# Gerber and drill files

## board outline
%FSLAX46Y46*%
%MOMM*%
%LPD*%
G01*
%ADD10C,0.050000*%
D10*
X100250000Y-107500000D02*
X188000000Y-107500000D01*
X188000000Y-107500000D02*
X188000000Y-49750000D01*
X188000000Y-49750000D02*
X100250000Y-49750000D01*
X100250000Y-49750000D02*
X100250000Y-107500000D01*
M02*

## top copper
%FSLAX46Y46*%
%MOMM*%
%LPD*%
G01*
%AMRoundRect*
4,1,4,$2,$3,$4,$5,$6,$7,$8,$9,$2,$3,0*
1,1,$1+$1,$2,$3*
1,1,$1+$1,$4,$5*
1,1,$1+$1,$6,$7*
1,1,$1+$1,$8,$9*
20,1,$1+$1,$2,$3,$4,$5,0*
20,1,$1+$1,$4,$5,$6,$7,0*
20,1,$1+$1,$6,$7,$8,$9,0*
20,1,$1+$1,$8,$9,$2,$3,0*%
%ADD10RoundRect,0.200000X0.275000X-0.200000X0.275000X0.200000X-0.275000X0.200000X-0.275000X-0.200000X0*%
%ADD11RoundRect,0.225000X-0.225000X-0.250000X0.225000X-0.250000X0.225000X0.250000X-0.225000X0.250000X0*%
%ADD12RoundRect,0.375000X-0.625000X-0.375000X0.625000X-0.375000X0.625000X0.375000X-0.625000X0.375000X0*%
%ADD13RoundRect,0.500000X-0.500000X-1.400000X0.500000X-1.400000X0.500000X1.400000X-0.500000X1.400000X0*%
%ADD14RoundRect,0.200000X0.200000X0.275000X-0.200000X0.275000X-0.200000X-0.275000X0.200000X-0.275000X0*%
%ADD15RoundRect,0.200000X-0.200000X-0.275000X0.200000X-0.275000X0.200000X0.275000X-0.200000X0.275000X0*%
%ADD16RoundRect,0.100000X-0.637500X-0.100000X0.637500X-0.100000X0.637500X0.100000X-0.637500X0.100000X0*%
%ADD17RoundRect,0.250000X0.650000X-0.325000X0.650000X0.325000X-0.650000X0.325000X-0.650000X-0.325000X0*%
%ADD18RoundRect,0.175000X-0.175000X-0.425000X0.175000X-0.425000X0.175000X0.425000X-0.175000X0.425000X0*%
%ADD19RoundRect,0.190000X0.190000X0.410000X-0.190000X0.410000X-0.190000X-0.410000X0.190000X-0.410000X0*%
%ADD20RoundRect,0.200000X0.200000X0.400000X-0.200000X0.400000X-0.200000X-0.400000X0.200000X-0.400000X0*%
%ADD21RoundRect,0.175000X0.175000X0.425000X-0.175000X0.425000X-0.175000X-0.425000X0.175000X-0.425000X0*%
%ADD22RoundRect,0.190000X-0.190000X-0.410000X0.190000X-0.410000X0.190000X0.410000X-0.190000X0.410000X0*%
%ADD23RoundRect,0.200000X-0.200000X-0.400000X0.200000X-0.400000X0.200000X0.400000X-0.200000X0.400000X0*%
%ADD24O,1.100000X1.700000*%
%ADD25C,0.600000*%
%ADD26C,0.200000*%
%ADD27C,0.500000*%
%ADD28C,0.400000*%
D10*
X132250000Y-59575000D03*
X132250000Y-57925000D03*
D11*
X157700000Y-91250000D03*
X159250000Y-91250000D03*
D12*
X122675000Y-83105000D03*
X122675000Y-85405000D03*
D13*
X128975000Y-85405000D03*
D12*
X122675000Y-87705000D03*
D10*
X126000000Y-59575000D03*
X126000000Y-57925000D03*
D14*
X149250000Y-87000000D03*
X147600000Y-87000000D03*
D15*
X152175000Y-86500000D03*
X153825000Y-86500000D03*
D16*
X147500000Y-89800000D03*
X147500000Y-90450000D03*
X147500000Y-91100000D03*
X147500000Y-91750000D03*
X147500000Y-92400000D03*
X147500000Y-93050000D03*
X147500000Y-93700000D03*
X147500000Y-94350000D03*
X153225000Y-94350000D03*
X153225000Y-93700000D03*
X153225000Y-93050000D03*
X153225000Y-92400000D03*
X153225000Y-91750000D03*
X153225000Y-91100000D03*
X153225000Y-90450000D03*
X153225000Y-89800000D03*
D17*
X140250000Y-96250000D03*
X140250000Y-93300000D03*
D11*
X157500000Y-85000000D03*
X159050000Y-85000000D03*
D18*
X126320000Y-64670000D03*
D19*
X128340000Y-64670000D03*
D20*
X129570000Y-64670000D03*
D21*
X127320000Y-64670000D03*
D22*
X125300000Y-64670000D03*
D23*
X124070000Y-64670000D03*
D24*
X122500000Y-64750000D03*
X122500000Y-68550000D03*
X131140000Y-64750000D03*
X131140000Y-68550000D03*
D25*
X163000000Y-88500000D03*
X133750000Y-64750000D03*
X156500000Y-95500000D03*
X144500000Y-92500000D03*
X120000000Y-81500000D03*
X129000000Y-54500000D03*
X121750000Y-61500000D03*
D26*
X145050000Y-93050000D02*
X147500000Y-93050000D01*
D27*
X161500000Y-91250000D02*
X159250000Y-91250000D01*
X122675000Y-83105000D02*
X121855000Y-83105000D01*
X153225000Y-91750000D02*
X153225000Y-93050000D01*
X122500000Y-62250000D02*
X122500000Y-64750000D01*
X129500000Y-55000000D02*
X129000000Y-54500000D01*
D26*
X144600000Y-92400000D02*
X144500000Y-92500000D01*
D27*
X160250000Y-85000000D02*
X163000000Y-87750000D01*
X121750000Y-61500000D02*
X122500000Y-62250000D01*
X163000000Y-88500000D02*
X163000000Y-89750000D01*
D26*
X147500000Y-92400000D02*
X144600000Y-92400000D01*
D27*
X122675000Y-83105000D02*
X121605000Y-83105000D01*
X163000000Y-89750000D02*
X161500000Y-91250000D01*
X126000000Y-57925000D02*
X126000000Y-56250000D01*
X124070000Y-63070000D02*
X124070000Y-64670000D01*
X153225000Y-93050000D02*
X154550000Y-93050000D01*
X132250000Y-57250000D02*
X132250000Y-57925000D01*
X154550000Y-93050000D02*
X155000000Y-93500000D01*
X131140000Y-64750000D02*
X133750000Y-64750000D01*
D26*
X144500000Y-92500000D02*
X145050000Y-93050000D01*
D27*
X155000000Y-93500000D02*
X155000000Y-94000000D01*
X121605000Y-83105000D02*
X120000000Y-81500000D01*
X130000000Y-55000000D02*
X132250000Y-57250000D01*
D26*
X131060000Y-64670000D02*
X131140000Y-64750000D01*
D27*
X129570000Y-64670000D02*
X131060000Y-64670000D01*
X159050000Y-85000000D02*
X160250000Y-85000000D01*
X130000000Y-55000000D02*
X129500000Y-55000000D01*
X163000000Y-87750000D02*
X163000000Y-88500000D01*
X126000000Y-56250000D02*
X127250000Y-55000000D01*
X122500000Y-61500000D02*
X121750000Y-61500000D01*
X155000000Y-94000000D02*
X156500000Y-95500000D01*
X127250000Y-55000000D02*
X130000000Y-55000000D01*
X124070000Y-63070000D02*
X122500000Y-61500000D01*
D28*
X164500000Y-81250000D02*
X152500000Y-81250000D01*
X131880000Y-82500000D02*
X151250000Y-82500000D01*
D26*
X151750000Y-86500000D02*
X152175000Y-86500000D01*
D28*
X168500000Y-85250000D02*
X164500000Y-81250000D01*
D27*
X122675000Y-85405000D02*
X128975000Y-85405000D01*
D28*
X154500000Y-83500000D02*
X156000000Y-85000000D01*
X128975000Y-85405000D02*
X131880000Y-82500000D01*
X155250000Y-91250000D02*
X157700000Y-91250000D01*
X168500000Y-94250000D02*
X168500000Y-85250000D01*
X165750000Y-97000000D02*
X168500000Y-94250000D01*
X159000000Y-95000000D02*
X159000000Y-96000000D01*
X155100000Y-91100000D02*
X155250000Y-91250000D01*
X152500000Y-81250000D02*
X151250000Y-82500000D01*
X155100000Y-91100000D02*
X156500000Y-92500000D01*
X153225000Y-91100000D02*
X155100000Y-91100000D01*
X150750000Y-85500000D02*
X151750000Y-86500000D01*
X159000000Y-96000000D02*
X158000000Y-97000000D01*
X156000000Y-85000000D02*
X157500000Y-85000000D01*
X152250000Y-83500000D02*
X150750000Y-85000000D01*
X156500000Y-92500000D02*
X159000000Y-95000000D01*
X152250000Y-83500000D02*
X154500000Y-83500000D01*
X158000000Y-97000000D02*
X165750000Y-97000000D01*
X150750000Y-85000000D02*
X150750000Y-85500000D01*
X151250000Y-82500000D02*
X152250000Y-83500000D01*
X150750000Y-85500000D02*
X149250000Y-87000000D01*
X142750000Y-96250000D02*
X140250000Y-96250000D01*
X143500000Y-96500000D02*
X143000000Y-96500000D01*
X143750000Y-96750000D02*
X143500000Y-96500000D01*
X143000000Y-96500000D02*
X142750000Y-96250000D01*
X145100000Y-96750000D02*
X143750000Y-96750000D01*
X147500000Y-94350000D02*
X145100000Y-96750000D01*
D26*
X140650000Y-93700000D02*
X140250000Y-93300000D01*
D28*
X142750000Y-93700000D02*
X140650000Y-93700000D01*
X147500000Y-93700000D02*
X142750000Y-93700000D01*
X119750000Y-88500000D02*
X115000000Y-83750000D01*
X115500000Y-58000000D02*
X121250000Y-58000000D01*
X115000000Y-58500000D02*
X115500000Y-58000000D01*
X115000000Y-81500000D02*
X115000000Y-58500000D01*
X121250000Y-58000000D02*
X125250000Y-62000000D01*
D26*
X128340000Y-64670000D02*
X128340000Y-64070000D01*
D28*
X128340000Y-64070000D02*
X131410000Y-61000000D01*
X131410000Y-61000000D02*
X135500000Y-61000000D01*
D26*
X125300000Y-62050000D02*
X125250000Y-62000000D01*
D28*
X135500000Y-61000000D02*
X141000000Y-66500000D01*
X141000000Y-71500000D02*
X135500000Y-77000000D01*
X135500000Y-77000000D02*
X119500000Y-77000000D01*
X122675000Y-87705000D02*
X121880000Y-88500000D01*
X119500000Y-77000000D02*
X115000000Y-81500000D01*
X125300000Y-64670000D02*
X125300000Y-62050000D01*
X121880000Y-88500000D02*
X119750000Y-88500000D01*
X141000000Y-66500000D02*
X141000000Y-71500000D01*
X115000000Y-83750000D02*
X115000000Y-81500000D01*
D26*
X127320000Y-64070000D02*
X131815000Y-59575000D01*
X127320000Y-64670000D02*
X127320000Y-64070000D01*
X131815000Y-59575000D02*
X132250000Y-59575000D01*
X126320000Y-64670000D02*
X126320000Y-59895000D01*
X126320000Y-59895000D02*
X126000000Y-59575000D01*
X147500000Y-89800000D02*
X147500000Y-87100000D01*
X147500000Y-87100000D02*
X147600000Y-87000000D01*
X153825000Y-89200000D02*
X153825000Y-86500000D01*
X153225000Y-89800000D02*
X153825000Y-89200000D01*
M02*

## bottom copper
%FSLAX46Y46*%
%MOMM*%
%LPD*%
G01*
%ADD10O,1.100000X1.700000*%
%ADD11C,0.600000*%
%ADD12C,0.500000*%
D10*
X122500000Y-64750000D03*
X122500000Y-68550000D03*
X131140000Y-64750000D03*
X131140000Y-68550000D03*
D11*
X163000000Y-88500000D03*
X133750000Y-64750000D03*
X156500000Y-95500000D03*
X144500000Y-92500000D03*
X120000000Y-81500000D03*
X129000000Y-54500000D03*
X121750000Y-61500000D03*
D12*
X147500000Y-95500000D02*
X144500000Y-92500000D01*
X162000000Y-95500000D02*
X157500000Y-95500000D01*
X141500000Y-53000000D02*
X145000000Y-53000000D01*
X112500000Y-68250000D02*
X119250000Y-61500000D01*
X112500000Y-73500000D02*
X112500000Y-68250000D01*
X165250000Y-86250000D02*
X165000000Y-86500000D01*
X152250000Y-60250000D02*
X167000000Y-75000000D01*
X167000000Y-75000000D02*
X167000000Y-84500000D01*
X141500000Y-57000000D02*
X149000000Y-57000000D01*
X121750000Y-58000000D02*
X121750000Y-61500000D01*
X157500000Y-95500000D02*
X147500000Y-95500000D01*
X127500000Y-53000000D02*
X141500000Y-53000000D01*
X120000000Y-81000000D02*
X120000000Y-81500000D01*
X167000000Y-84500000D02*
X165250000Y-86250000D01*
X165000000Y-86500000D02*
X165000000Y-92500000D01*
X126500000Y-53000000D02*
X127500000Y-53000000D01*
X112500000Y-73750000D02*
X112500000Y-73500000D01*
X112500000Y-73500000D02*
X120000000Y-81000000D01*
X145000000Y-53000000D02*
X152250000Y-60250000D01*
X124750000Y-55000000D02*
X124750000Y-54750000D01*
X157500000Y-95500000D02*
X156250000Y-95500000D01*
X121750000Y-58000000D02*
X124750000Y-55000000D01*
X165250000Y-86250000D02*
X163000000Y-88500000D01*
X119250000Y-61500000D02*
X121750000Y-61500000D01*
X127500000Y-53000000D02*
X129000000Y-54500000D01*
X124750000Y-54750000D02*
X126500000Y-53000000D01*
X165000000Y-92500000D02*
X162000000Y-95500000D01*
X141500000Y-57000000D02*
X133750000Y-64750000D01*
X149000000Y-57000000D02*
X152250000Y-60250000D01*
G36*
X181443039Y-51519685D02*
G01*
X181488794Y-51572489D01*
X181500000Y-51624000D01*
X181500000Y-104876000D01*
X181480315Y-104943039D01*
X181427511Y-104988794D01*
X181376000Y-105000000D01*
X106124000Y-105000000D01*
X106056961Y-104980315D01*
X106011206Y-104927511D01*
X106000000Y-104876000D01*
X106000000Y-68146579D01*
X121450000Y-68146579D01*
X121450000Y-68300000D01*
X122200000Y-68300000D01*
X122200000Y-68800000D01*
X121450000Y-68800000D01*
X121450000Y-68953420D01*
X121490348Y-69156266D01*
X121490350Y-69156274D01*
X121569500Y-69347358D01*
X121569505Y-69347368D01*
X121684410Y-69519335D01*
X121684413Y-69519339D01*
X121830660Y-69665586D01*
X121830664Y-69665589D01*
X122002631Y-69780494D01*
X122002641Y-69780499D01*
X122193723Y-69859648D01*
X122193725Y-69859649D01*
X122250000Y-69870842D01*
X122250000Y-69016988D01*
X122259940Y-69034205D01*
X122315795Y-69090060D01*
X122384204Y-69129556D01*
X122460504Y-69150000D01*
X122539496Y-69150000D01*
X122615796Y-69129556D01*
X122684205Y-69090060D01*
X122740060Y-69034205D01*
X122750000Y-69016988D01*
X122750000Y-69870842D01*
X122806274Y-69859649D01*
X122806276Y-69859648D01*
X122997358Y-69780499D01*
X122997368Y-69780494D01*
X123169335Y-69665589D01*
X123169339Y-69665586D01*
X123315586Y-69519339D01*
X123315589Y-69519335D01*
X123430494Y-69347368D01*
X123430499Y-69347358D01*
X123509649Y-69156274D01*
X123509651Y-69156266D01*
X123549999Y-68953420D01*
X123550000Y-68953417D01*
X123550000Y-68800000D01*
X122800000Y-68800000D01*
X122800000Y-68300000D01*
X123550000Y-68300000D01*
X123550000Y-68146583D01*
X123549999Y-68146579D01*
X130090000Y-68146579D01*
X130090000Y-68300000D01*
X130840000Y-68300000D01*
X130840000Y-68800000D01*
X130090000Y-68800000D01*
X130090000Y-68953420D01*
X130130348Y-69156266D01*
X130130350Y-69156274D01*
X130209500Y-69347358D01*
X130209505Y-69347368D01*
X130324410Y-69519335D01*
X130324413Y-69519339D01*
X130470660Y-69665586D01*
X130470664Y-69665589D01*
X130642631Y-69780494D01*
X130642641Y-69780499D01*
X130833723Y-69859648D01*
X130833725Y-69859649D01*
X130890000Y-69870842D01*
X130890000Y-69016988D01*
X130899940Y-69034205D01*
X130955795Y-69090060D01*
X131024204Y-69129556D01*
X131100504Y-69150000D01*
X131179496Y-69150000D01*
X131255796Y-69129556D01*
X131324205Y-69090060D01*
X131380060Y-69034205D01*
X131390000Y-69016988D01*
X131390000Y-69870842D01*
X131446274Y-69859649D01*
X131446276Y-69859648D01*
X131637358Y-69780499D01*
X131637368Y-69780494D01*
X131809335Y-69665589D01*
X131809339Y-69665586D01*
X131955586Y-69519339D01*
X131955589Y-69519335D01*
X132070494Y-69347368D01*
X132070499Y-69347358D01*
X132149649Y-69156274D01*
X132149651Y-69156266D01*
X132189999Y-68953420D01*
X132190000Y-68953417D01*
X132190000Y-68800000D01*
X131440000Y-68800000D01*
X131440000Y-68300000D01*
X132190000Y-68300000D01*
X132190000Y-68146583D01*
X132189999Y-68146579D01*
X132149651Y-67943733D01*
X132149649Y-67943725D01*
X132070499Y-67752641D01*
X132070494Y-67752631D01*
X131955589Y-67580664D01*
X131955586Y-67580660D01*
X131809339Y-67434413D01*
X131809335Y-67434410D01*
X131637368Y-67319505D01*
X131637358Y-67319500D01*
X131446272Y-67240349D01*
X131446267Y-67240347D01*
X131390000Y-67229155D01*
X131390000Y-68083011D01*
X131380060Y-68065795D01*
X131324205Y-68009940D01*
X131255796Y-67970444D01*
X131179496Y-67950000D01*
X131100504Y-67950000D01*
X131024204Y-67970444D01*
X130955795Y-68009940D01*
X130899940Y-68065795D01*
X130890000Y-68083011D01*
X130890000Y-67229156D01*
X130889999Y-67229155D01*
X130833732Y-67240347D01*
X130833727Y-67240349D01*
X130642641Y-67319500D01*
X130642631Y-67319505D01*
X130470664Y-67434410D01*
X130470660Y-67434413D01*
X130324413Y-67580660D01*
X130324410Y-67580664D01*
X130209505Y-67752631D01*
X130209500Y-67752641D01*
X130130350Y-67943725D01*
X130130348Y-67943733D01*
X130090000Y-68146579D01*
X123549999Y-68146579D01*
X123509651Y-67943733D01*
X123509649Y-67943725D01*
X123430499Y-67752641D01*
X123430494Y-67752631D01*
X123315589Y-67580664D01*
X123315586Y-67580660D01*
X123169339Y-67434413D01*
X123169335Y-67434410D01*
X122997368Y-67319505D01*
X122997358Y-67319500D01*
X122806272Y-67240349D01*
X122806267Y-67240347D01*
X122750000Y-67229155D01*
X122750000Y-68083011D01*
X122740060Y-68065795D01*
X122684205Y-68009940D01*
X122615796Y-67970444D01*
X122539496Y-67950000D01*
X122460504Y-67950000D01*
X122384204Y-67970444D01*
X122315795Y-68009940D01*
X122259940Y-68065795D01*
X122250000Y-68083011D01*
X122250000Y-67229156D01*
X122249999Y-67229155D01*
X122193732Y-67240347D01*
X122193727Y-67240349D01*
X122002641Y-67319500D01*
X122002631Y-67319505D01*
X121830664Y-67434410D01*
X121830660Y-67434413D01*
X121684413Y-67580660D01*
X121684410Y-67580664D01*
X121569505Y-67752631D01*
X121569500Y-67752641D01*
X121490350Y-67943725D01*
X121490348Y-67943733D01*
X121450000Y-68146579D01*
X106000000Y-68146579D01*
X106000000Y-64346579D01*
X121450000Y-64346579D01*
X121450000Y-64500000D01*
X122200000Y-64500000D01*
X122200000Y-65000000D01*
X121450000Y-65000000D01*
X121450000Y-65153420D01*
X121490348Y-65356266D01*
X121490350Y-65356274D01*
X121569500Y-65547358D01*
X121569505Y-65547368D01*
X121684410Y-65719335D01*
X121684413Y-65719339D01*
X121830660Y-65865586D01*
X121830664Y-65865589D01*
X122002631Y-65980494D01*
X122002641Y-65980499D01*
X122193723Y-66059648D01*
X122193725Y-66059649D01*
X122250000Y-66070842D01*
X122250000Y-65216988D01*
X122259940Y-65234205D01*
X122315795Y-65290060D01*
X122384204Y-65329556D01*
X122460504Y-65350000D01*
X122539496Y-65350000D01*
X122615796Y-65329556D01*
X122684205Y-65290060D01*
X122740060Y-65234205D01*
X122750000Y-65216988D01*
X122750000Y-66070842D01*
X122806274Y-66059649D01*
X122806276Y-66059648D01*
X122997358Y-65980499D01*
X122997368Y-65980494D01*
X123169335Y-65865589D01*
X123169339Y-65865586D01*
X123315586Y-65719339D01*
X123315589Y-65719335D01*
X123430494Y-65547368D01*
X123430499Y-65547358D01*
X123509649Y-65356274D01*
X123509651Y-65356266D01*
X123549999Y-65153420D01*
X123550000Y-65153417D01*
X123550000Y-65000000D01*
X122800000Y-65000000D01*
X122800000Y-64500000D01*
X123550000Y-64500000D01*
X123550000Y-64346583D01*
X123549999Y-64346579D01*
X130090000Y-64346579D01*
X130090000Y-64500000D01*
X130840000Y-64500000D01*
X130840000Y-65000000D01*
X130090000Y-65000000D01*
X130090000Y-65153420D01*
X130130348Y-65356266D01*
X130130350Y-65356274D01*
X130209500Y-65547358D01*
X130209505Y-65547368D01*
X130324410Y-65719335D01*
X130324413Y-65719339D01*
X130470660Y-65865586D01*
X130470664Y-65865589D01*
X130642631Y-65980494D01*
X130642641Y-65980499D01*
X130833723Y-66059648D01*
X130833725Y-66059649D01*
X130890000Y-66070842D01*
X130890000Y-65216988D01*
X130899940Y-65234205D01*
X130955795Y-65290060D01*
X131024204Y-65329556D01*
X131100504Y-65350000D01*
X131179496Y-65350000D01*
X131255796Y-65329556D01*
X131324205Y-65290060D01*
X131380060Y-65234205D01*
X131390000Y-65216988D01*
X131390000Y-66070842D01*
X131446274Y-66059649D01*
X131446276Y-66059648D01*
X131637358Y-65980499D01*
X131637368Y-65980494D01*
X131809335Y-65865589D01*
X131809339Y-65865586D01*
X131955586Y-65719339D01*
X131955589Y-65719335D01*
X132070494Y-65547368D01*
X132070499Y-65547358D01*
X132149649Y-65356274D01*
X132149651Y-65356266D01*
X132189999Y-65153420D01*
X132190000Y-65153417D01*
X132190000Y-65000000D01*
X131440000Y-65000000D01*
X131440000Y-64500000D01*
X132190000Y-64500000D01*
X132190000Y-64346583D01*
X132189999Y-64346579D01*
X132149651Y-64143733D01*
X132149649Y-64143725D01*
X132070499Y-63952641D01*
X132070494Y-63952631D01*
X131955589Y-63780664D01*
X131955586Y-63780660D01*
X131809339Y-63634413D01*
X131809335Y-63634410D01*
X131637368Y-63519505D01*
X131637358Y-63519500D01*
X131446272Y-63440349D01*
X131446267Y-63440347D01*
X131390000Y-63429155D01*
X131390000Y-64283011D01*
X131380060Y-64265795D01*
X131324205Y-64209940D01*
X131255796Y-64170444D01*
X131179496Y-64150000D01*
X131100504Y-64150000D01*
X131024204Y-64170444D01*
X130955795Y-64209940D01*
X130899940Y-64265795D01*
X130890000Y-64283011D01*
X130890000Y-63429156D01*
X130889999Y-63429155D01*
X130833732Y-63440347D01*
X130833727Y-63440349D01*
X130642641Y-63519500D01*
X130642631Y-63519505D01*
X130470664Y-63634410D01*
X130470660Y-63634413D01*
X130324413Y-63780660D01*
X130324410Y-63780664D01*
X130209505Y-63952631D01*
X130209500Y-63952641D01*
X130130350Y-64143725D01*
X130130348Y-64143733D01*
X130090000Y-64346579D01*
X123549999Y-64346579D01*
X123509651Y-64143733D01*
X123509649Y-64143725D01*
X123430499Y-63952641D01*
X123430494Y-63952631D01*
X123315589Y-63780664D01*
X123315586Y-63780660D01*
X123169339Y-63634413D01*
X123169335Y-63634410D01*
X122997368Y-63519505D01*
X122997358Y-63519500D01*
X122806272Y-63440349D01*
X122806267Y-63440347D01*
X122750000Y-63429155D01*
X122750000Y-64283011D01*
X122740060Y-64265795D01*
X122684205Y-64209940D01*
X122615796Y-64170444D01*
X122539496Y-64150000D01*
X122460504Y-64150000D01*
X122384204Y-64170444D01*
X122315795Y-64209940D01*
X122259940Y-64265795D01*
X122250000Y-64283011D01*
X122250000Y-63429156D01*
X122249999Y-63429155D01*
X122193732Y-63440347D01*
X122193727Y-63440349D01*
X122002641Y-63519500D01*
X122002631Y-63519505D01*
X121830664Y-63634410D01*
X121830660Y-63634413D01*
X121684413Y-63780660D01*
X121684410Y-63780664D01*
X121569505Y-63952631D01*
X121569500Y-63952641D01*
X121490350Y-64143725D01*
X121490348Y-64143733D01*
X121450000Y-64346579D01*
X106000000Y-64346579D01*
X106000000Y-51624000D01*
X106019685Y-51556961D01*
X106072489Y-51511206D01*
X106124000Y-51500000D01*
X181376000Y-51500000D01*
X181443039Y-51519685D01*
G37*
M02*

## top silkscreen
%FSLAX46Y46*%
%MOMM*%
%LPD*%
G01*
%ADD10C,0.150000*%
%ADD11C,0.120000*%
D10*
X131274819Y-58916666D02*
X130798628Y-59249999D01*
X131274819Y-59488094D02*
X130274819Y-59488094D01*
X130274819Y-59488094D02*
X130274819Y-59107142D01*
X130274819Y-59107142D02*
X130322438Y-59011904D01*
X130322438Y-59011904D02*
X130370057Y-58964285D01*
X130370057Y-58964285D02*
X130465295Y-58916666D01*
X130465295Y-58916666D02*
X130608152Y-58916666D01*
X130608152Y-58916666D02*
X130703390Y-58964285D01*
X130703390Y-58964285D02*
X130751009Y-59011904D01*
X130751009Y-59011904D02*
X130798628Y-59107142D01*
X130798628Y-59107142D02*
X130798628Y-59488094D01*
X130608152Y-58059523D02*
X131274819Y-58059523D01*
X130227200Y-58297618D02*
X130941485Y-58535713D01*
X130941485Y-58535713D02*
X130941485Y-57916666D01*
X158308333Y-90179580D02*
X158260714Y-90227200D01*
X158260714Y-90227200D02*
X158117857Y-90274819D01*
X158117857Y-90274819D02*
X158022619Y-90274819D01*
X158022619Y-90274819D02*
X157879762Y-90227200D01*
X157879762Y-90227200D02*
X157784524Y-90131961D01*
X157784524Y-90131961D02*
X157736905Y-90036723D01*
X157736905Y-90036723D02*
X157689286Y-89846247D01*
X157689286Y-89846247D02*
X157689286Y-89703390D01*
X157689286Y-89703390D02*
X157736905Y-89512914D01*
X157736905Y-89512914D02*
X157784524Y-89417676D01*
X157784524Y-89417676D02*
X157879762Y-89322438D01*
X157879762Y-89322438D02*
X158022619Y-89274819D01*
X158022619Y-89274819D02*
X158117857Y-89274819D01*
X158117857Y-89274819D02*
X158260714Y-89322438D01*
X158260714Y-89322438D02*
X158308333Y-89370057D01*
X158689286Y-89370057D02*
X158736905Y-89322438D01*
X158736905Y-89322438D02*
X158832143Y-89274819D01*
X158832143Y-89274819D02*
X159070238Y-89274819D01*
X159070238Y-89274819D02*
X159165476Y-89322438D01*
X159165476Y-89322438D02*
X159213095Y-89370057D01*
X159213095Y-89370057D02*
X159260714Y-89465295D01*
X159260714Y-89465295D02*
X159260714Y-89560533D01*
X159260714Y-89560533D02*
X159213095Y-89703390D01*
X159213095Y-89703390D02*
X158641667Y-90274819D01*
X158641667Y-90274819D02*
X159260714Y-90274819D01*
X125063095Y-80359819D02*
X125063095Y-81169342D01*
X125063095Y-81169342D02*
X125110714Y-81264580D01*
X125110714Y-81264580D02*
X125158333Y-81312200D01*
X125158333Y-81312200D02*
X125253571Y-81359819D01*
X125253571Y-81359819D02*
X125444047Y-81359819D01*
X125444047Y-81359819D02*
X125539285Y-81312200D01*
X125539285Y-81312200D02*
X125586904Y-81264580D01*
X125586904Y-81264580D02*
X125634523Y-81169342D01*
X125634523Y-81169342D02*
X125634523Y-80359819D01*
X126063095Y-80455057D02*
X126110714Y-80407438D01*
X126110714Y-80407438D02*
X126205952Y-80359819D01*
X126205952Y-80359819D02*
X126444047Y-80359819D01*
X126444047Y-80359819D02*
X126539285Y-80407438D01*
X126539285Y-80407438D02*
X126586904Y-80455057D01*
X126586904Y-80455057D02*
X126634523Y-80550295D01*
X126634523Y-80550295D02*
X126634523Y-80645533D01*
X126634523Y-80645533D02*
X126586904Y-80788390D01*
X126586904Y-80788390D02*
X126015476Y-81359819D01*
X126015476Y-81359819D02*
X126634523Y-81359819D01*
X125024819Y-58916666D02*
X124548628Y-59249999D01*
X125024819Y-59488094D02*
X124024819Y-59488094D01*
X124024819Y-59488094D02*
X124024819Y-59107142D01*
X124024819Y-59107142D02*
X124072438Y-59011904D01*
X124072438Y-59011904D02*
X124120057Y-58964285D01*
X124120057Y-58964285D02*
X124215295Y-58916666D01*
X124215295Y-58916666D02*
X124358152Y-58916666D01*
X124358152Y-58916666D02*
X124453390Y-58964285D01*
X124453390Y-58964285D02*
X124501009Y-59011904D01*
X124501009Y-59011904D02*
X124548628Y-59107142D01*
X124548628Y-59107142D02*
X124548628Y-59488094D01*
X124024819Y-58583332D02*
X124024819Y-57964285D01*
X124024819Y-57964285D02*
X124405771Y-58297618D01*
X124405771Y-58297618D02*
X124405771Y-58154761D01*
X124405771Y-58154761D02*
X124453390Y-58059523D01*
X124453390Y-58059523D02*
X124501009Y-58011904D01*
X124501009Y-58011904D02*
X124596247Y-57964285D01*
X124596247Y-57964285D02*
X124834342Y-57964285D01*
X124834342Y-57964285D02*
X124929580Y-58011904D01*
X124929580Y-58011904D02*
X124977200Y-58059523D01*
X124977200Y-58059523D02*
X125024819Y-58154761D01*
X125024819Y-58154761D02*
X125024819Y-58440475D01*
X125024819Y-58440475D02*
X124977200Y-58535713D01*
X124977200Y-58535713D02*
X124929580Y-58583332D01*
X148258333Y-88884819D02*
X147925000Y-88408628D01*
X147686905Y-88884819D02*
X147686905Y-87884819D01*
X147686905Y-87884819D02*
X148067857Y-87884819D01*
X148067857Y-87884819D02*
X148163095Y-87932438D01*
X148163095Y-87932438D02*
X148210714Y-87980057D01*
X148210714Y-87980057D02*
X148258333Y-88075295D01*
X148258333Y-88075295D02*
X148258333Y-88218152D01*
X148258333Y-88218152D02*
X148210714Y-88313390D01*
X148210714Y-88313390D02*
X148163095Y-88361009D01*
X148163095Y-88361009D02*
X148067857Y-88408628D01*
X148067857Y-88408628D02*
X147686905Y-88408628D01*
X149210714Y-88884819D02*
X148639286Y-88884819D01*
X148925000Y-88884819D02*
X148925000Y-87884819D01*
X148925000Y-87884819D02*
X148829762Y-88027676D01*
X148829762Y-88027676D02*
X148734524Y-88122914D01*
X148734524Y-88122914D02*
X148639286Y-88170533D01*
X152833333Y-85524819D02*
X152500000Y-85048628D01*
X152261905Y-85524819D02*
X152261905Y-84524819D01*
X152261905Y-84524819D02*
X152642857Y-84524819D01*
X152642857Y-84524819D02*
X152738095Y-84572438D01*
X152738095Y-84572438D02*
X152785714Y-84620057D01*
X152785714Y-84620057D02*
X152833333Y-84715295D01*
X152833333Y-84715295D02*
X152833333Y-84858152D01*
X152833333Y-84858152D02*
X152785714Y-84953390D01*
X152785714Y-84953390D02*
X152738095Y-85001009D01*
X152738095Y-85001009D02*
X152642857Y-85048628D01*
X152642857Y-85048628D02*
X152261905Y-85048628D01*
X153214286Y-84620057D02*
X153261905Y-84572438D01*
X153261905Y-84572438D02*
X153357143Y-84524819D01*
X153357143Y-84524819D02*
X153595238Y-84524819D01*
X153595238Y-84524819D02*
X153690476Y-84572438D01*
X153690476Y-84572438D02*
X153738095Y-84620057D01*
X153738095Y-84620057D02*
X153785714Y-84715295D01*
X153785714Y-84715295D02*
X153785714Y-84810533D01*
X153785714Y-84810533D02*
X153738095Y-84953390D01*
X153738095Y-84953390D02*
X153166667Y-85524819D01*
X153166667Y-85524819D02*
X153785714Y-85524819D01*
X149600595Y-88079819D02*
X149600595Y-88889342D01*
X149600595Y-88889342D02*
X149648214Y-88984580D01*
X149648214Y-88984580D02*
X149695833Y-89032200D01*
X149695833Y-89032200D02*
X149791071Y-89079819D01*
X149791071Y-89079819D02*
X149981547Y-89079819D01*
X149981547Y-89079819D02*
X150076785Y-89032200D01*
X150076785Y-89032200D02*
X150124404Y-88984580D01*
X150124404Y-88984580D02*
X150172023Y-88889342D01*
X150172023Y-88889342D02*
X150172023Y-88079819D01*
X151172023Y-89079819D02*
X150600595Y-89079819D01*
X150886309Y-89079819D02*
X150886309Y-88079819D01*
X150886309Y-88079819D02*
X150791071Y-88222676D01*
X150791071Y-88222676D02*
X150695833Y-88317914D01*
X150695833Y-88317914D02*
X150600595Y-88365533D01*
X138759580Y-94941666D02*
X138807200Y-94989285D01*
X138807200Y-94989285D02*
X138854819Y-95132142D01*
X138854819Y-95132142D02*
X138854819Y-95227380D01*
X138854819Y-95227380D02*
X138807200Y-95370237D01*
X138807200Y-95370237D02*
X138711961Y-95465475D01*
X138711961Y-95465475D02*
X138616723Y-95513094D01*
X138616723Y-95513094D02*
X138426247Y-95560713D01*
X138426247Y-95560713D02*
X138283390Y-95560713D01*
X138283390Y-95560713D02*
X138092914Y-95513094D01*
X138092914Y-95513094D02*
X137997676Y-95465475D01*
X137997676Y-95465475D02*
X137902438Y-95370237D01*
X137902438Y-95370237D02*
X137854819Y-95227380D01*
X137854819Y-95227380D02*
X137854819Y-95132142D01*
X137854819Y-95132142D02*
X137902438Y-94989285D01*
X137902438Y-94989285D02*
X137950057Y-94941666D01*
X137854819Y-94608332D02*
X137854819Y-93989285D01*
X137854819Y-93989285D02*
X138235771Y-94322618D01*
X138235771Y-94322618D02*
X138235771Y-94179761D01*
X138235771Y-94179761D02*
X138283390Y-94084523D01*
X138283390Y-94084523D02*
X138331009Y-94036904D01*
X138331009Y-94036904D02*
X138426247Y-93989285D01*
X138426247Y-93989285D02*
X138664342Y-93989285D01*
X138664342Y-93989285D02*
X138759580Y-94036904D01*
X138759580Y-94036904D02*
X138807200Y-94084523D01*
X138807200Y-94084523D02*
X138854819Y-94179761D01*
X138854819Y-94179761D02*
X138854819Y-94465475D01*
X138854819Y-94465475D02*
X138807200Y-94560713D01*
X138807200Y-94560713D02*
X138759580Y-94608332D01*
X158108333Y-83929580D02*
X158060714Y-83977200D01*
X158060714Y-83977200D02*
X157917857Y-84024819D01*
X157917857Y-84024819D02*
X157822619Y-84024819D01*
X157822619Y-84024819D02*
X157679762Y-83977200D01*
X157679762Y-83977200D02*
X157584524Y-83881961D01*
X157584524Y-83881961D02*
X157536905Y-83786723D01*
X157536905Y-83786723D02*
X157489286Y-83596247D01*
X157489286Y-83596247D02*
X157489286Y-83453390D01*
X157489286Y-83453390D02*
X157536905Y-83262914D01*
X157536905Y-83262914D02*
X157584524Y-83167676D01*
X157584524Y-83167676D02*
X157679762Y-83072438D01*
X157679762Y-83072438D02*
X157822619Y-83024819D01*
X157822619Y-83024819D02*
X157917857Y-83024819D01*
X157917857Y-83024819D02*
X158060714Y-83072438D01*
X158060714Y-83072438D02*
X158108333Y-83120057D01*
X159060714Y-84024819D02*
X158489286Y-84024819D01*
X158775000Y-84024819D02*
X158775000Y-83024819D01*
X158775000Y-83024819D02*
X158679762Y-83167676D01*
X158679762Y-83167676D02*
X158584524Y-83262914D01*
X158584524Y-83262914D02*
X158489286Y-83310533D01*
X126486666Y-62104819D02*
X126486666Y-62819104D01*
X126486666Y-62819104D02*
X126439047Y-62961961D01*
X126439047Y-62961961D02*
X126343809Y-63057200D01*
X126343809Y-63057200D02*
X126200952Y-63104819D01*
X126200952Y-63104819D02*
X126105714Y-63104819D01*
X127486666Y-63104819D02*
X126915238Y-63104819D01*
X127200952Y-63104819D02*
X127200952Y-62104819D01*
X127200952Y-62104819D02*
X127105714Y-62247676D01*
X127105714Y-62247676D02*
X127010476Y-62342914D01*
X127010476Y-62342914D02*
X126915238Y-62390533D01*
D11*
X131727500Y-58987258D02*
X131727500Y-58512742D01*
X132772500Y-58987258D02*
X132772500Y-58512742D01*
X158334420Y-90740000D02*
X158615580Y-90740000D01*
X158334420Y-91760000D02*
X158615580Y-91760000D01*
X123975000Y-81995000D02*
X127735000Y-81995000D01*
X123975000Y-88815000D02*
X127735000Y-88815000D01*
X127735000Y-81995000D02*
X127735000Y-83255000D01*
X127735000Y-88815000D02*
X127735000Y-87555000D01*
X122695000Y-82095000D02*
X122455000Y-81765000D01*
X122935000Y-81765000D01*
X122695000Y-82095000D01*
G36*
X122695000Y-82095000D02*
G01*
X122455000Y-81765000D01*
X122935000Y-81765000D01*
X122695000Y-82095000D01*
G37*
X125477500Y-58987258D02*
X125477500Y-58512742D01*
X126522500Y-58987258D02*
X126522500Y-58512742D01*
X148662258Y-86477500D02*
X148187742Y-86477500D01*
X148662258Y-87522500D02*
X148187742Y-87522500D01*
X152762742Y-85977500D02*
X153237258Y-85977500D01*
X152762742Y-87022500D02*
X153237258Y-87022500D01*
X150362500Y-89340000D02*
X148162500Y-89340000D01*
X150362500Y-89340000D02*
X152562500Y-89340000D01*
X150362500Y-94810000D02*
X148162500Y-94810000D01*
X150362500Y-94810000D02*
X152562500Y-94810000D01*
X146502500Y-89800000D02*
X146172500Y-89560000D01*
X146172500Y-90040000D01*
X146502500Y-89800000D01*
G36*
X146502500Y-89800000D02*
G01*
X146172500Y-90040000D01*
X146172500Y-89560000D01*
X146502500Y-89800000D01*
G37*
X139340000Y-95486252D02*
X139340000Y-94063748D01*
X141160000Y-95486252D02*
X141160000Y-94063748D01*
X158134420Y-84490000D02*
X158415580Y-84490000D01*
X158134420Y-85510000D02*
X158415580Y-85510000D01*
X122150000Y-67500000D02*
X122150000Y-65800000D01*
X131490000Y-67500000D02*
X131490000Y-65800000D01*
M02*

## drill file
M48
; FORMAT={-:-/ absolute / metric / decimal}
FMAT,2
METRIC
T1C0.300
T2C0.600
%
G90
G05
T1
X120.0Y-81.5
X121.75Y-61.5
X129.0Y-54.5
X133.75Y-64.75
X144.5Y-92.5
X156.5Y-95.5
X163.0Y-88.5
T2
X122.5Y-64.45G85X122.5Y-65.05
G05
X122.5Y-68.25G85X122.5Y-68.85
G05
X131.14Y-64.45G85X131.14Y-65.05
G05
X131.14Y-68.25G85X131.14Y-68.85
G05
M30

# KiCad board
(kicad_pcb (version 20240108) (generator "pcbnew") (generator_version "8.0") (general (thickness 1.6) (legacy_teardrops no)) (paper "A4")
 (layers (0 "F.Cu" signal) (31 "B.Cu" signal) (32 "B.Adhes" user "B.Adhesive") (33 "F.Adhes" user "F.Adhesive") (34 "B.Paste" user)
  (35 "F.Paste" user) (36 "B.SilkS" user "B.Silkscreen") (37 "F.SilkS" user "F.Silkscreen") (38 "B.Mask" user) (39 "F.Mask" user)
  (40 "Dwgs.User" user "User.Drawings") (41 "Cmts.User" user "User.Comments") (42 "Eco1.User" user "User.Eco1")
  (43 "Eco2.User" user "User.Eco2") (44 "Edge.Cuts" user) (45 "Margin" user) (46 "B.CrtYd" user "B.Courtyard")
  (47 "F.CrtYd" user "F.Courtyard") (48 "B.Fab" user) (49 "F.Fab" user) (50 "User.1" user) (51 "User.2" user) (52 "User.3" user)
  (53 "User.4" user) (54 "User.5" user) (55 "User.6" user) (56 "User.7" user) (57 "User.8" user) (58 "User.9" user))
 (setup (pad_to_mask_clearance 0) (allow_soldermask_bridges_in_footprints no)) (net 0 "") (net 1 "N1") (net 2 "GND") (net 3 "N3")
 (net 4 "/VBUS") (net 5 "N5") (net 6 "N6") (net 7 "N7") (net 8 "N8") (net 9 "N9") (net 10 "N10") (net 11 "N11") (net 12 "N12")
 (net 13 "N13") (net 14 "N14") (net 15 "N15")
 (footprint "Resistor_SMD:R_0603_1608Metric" (layer "F.Cu") (at 132.25 58.75 90)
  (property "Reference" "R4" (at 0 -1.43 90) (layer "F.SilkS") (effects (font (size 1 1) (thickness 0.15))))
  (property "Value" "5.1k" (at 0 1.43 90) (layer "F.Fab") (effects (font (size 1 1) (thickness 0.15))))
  (fp_line (start -0.237258 -0.5225) (end 0.237258 -0.5225) (stroke (width 0.12) (type solid)) (layer "F.SilkS"))
  (fp_line (start -0.237258 0.5225) (end 0.237258 0.5225) (stroke (width 0.12) (type solid)) (layer "F.SilkS"))
  (pad "1" smd roundrect (at -0.825 0 90) (size 0.8 0.95) (layers "F.Cu" "F.Paste" "F.Mask") (roundrect_rratio 0.25) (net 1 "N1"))
  (pad "2" smd roundrect (at 0.825 0 90) (size 0.8 0.95) (layers "F.Cu" "F.Paste" "F.Mask") (roundrect_rratio 0.25) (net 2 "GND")))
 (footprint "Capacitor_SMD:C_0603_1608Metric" (layer "F.Cu") (at 158.475 91.25)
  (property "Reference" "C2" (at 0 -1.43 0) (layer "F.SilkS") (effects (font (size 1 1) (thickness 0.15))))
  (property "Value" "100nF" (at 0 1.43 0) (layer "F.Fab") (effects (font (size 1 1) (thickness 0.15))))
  (fp_line (start -0.14058 -0.51) (end 0.14058 -0.51) (stroke (width 0.12) (type solid)) (layer "F.SilkS"))
  (fp_line (start -0.14058 0.51) (end 0.14058 0.51) (stroke (width 0.12) (type solid)) (layer "F.SilkS"))
  (pad "1" smd roundrect (at -0.775 0) (size 0.9 0.95) (layers "F.Cu" "F.Paste" "F.Mask") (roundrect_rratio 0.25) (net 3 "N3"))
  (pad "2" smd roundrect (at 0.775 0) (size 0.9 0.95) (layers "F.Cu" "F.Paste" "F.Mask") (roundrect_rratio 0.25) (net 2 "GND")))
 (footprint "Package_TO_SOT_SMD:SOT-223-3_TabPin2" (layer "F.Cu") (at 125.825 85.405)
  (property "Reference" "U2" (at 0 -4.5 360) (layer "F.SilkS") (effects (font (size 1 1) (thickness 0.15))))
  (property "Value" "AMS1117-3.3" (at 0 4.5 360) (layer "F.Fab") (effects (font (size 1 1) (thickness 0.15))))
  (fp_line (start -1.85 -3.41) (end 1.91 -3.41) (stroke (width 0.12) (type solid)) (layer "F.SilkS"))
  (fp_line (start -1.85 3.41) (end 1.91 3.41) (stroke (width 0.12) (type solid)) (layer "F.SilkS"))
  (fp_line (start 1.91 -3.41) (end 1.91 -2.15) (stroke (width 0.12) (type solid)) (layer "F.SilkS"))
  (fp_line (start 1.91 3.41) (end 1.91 2.15) (stroke (width 0.12) (type solid)) (layer "F.SilkS"))
  (fp_poly
   (pts (xy -3.13 -3.31) (xy -3.37 -3.64) (xy -2.89 -3.64) (xy -3.13 -3.31)) (stroke (width 0.12) (type solid)) (fill solid)
   (layer "F.SilkS"))
  (pad "1" smd roundrect (at -3.15 -2.3) (size 2 1.5) (layers "F.Cu" "F.Paste" "F.Mask") (roundrect_rratio 0.25) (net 2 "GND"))
  (pad "2" smd roundrect (at -3.15 0) (size 2 1.5) (layers "F.Cu" "F.Paste" "F.Mask") (roundrect_rratio 0.25) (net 3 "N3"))
  (pad "2" smd roundrect (at 3.15 0) (size 2 3.8) (layers "F.Cu" "F.Paste" "F.Mask") (roundrect_rratio 0.25) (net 3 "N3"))
  (pad "3" smd roundrect (at -3.15 2.3) (size 2 1.5) (layers "F.Cu" "F.Paste" "F.Mask") (roundrect_rratio 0.25) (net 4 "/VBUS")))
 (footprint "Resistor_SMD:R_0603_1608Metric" (layer "F.Cu") (at 126 58.75 90)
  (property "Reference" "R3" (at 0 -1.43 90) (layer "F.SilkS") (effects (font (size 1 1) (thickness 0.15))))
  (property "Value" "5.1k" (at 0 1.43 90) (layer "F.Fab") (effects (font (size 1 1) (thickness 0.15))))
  (fp_line (start -0.237258 -0.5225) (end 0.237258 -0.5225) (stroke (width 0.12) (type solid)) (layer "F.SilkS"))
  (fp_line (start -0.237258 0.5225) (end 0.237258 0.5225) (stroke (width 0.12) (type solid)) (layer "F.SilkS"))
  (pad "1" smd roundrect (at -0.825 0 90) (size 0.8 0.95) (layers "F.Cu" "F.Paste" "F.Mask") (roundrect_rratio 0.25) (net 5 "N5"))
  (pad "2" smd roundrect (at 0.825 0 90) (size 0.8 0.95) (layers "F.Cu" "F.Paste" "F.Mask") (roundrect_rratio 0.25) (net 2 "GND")))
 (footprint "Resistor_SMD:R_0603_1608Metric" (layer "F.Cu") (at 148.425 87 180)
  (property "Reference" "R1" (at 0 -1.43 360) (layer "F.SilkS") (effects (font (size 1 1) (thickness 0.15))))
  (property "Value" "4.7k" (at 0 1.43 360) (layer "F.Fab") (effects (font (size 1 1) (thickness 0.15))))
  (fp_line (start -0.237258 0.5225) (end 0.237258 0.5225) (stroke (width 0.12) (type solid)) (layer "F.SilkS"))
  (fp_line (start -0.237258 -0.5225) (end 0.237258 -0.5225) (stroke (width 0.12) (type solid)) (layer "F.SilkS"))
  (pad "1" smd roundrect (at -0.825 0 180) (size 0.8 0.95) (layers "F.Cu" "F.Paste" "F.Mask") (roundrect_rratio 0.25) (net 3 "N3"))
  (pad "2" smd roundrect (at 0.825 0 180) (size 0.8 0.95) (layers "F.Cu" "F.Paste" "F.Mask") (roundrect_rratio 0.25) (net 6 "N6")))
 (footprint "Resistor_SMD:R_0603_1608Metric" (layer "F.Cu") (at 153 86.5)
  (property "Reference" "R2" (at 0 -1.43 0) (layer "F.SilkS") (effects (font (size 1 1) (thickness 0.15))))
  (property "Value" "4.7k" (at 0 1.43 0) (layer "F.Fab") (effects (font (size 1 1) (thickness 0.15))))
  (fp_line (start -0.237258 -0.5225) (end 0.237258 -0.5225) (stroke (width 0.12) (type solid)) (layer "F.SilkS"))
  (fp_line (start -0.237258 0.5225) (end 0.237258 0.5225) (stroke (width 0.12) (type solid)) (layer "F.SilkS"))
  (pad "1" smd roundrect (at -0.825 0) (size 0.8 0.95) (layers "F.Cu" "F.Paste" "F.Mask") (roundrect_rratio 0.25) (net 3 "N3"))
  (pad "2" smd roundrect (at 0.825 0) (size 0.8 0.95) (layers "F.Cu" "F.Paste" "F.Mask") (roundrect_rratio 0.25) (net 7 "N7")))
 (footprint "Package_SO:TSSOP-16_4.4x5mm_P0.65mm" (layer "F.Cu") (at 150.3625 92.075)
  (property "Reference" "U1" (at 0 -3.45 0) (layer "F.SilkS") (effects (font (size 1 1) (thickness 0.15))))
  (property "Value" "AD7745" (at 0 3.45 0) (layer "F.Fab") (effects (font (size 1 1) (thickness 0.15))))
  (fp_line (start 0 -2.735) (end -2.2 -2.735) (stroke (width 0.12) (type solid)) (layer "F.SilkS"))
  (fp_line (start 0 -2.735) (end 2.2 -2.735) (stroke (width 0.12) (type solid)) (layer "F.SilkS"))
  (fp_line (start 0 2.735) (end -2.2 2.735) (stroke (width 0.12) (type solid)) (layer "F.SilkS"))
  (fp_line (start 0 2.735) (end 2.2 2.735) (stroke (width 0.12) (type solid)) (layer "F.SilkS"))
  (fp_poly
   (pts (xy -3.86 -2.275) (xy -4.19 -2.515) (xy -4.19 -2.035) (xy -3.86 -2.275)) (stroke (width 0.12) (type solid)) (fill solid)
   (layer "F.SilkS"))
  (pad "1" smd roundrect (at -2.8625 -2.275) (size 1.475 0.4) (layers "F.Cu" "F.Paste" "F.Mask") (roundrect_rratio 0.25) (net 6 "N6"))
  (pad "2" smd roundrect (at -2.8625 -1.625) (size 1.475 0.4) (layers "F.Cu" "F.Paste" "F.Mask") (roundrect_rratio 0.25) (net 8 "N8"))
  (pad "3" smd roundrect (at -2.8625 -0.975) (size 1.475 0.4) (layers "F.Cu" "F.Paste" "F.Mask") (roundrect_rratio 0.25) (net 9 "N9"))
  (pad "4" smd roundrect (at -2.8625 -0.325) (size 1.475 0.4) (layers "F.Cu" "F.Paste" "F.Mask") (roundrect_rratio 0.25) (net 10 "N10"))
  (pad "5" smd roundrect (at -2.8625 0.325) (size 1.475 0.4) (layers "F.Cu" "F.Paste" "F.Mask") (roundrect_rratio 0.25) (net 2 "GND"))
  (pad "6" smd roundrect (at -2.8625 0.975) (size 1.475 0.4) (layers "F.Cu" "F.Paste" "F.Mask") (roundrect_rratio 0.25) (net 2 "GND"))
  (pad "7" smd roundrect (at -2.8625 1.625) (size 1.475 0.4) (layers "F.Cu" "F.Paste" "F.Mask") (roundrect_rratio 0.25) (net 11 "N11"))
  (pad "8" smd roundrect (at -2.8625 2.275) (size 1.475 0.4) (layers "F.Cu" "F.Paste" "F.Mask") (roundrect_rratio 0.25) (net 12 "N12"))
  (pad "9" smd roundrect (at 2.8625 2.275) (size 1.475 0.4) (layers "F.Cu" "F.Paste" "F.Mask") (roundrect_rratio 0.25) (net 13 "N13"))
  (pad "10" smd roundrect (at 2.8625 1.625) (size 1.475 0.4) (layers "F.Cu" "F.Paste" "F.Mask") (roundrect_rratio 0.25) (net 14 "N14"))
  (pad "11" smd roundrect (at 2.8625 0.975) (size 1.475 0.4) (layers "F.Cu" "F.Paste" "F.Mask") (roundrect_rratio 0.25) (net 2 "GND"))
  (pad "12" smd roundrect (at 2.8625 0.325) (size 1.475 0.4) (layers "F.Cu" "F.Paste" "F.Mask") (roundrect_rratio 0.25) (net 2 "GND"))
  (pad "13" smd roundrect (at 2.8625 -0.325) (size 1.475 0.4) (layers "F.Cu" "F.Paste" "F.Mask") (roundrect_rratio 0.25) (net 2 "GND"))
  (pad "14" smd roundrect (at 2.8625 -0.975) (size 1.475 0.4) (layers "F.Cu" "F.Paste" "F.Mask") (roundrect_rratio 0.25) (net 3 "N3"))
  (pad "15" smd roundrect (at 2.8625 -1.625) (size 1.475 0.4) (layers "F.Cu" "F.Paste" "F.Mask") (roundrect_rratio 0.25) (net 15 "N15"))
  (pad "16" smd roundrect (at 2.8625 -2.275) (size 1.475 0.4) (layers "F.Cu" "F.Paste" "F.Mask") (roundrect_rratio 0.25) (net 7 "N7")))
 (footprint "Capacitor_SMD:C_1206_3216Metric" (layer "F.Cu") (at 140.25 94.775 90)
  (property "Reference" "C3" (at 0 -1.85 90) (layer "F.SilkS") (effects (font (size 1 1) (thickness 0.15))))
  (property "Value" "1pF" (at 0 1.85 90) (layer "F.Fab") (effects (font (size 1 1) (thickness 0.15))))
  (fp_line (start -0.711252 -0.91) (end 0.711252 -0.91) (stroke (width 0.12) (type solid)) (layer "F.SilkS"))
  (fp_line (start -0.711252 0.91) (end 0.711252 0.91) (stroke (width 0.12) (type solid)) (layer "F.SilkS"))
  (pad "1" smd roundrect (at -1.475 0 90) (size 1.15 1.8) (layers "F.Cu" "F.Paste" "F.Mask") (roundrect_rratio 0.217391) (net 12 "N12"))
  (pad "2" smd roundrect (at 1.475 0 90) (size 1.15 1.8) (layers "F.Cu" "F.Paste" "F.Mask") (roundrect_rratio 0.217391) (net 11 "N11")))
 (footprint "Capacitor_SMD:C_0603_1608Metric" (layer "F.Cu") (at 158.275 85)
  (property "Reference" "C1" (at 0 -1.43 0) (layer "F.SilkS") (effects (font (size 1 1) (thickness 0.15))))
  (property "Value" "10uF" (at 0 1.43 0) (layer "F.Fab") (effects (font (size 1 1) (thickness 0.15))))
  (fp_line (start -0.14058 -0.51) (end 0.14058 -0.51) (stroke (width 0.12) (type solid)) (layer "F.SilkS"))
  (fp_line (start -0.14058 0.51) (end 0.14058 0.51) (stroke (width 0.12) (type solid)) (layer "F.SilkS"))
  (pad "1" smd roundrect (at -0.775 0) (size 0.9 0.95) (layers "F.Cu" "F.Paste" "F.Mask") (roundrect_rratio 0.25) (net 3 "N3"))
  (pad "2" smd roundrect (at 0.775 0) (size 0.9 0.95) (layers "F.Cu" "F.Paste" "F.Mask") (roundrect_rratio 0.25) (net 2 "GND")))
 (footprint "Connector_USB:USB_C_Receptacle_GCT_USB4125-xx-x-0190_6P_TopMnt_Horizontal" (layer "F.Cu") (at 126.82 67.75)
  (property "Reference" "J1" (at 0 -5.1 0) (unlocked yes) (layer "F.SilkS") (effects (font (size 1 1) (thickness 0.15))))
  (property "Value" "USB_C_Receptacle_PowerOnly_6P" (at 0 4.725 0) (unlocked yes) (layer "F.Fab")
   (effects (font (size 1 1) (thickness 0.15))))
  (fp_line (start -4.67 -0.25) (end -4.67 -1.95) (stroke (width 0.12) (type solid)) (layer "F.SilkS"))
  (fp_line (start 4.67 -0.25) (end 4.67 -1.95) (stroke (width 0.12) (type solid)) (layer "F.SilkS"))
  (pad "A5" smd roundrect (at -0.5 -3.08) (size 0.7 1.2) (layers "F.Cu" "F.Paste" "F.Mask") (roundrect_rratio 0.25) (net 5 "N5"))
  (pad "A9" smd roundrect (at 1.52 -3.08 180) (size 0.76 1.2) (layers "F.Cu" "F.Paste" "F.Mask") (roundrect_rratio 0.25) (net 4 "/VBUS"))
  (pad "A12" smd roundrect (at 2.75 -3.08 180) (size 0.8 1.2) (layers "F.Cu" "F.Paste" "F.Mask") (roundrect_rratio 0.25) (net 2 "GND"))
  (pad "B5" smd roundrect (at 0.5 -3.08 180) (size 0.7 1.2) (layers "F.Cu" "F.Paste" "F.Mask") (roundrect_rratio 0.25) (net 1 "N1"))
  (pad "B9" smd roundrect (at -1.52 -3.08) (size 0.76 1.2) (layers "F.Cu" "F.Paste" "F.Mask") (roundrect_rratio 0.25) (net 4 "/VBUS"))
  (pad "B12" smd roundrect (at -2.75 -3.08) (size 0.8 1.2) (layers "F.Cu" "F.Paste" "F.Mask") (roundrect_rratio 0.25) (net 2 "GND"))
  (pad "S1" thru_hole oval (at -4.32 -3) (size 1.1 1.7) (drill oval 0.6 1.2) (layers "*.Cu" "*.Mask" "F.Paste") (remove_unused_layers no)
   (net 2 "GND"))
  (pad "S1" thru_hole oval (at -4.32 0.8) (size 1.1 1.7) (drill oval 0.6 1.2) (layers "*.Cu" "*.Mask" "F.Paste") (remove_unused_layers no)
   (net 2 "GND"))
  (pad "S1" thru_hole oval (at 4.32 -3) (size 1.1 1.7) (drill oval 0.6 1.2) (layers "*.Cu" "*.Mask" "F.Paste") (remove_unused_layers no)
   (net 2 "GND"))
  (pad "S1" thru_hole oval (at 4.32 0.8) (size 1.1 1.7) (drill oval 0.6 1.2) (layers "*.Cu" "*.Mask" "F.Paste") (remove_unused_layers no)
   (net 2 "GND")))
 (gr_line (start 100.25 107.5) (end 188 107.5) (stroke (width 0.05) (type default)) (layer "Edge.Cuts"))
 (gr_line (start 188 107.5) (end 188 49.75) (stroke (width 0.05) (type default)) (layer "Edge.Cuts"))
 (gr_line (start 188 49.75) (end 100.25 49.75) (stroke (width 0.05) (type default)) (layer "Edge.Cuts"))
 (gr_line (start 100.25 49.75) (end 100.25 107.5) (stroke (width 0.05) (type default)) (layer "Edge.Cuts"))
 (segment (start 145.05 93.05) (end 147.5 93.05) (width 0.2) (layer "F.Cu") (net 2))
 (segment (start 161.5 91.25) (end 159.25 91.25) (width 0.5) (layer "F.Cu") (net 2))
 (segment (start 122.675 83.105) (end 121.855 83.105) (width 0.5) (layer "F.Cu") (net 2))
 (segment (start 153.225 91.75) (end 153.225 93.05) (width 0.5) (layer "F.Cu") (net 2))
 (segment (start 122.5 62.25) (end 122.5 64.75) (width 0.5) (layer "F.Cu") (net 2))
 (segment (start 129.5 55) (end 129 54.5) (width 0.5) (layer "F.Cu") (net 2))
 (segment (start 144.6 92.4) (end 144.5 92.5) (width 0.2) (layer "F.Cu") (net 2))
 (segment (start 160.25 85) (end 163 87.75) (width 0.5) (layer "F.Cu") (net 2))
 (segment (start 121.75 61.5) (end 122.5 62.25) (width 0.5) (layer "F.Cu") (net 2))
 (segment (start 163 88.5) (end 163 89.75) (width 0.5) (layer "F.Cu") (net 2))
 (segment (start 147.5 92.4) (end 144.6 92.4) (width 0.2) (layer "F.Cu") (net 2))
 (segment (start 122.675 83.105) (end 121.605 83.105) (width 0.5) (layer "F.Cu") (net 2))
 (segment (start 163 89.75) (end 161.5 91.25) (width 0.5) (layer "F.Cu") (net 2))
 (segment (start 126 57.925) (end 126 56.25) (width 0.5) (layer "F.Cu") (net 2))
 (segment (start 124.07 63.07) (end 124.07 64.67) (width 0.5) (layer "F.Cu") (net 2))
 (segment (start 153.225 93.05) (end 154.55 93.05) (width 0.5) (layer "F.Cu") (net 2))
 (segment (start 132.25 57.25) (end 132.25 57.925) (width 0.5) (layer "F.Cu") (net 2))
 (segment (start 154.55 93.05) (end 155 93.5) (width 0.5) (layer "F.Cu") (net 2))
 (segment (start 131.14 64.75) (end 133.75 64.75) (width 0.5) (layer "F.Cu") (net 2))
 (segment (start 144.5 92.5) (end 145.05 93.05) (width 0.2) (layer "F.Cu") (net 2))
 (segment (start 155 93.5) (end 155 94) (width 0.5) (layer "F.Cu") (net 2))
 (segment (start 121.605 83.105) (end 120 81.5) (width 0.5) (layer "F.Cu") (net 2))
 (segment (start 130 55) (end 132.25 57.25) (width 0.5) (layer "F.Cu") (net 2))
 (segment (start 131.06 64.67) (end 131.14 64.75) (width 0.2) (layer "F.Cu") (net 2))
 (segment (start 129.57 64.67) (end 131.06 64.67) (width 0.5) (layer "F.Cu") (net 2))
 (segment (start 159.05 85) (end 160.25 85) (width 0.5) (layer "F.Cu") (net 2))
 (segment (start 130 55) (end 129.5 55) (width 0.5) (layer "F.Cu") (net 2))
 (segment (start 163 87.75) (end 163 88.5) (width 0.5) (layer "F.Cu") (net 2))
 (segment (start 126 56.25) (end 127.25 55) (width 0.5) (layer "F.Cu") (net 2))
 (segment (start 122.5 61.5) (end 121.75 61.5) (width 0.5) (layer "F.Cu") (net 2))
 (segment (start 155 94) (end 156.5 95.5) (width 0.5) (layer "F.Cu") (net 2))
 (segment (start 127.25 55) (end 130 55) (width 0.5) (layer "F.Cu") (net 2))
 (segment (start 124.07 63.07) (end 122.5 61.5) (width 0.5) (layer "F.Cu") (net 2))
 (via (at 163 88.5) (size 0.6) (drill 0.3) (layers "F.Cu" "B.Cu") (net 2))
 (via (at 133.75 64.75) (size 0.6) (drill 0.3) (layers "F.Cu" "B.Cu") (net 2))
 (via (at 156.5 95.5) (size 0.6) (drill 0.3) (layers "F.Cu" "B.Cu") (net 2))
 (via (at 144.5 92.5) (size 0.6) (drill 0.3) (layers "F.Cu" "B.Cu") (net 2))
 (via (at 120 81.5) (size 0.6) (drill 0.3) (layers "F.Cu" "B.Cu") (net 2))
 (via (at 129 54.5) (size 0.6) (drill 0.3) (layers "F.Cu" "B.Cu") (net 2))
 (via (at 121.75 61.5) (size 0.6) (drill 0.3) (layers "F.Cu" "B.Cu") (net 2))
 (segment (start 147.5 95.5) (end 144.5 92.5) (width 0.5) (layer "B.Cu") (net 2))
 (segment (start 162 95.5) (end 157.5 95.5) (width 0.5) (layer "B.Cu") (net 2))
 (segment (start 141.5 53) (end 145 53) (width 0.5) (layer "B.Cu") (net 2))
 (segment (start 112.5 68.25) (end 119.25 61.5) (width 0.5) (layer "B.Cu") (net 2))
 (segment (start 112.5 73.5) (end 112.5 68.25) (width 0.5) (layer "B.Cu") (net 2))
 (segment (start 165.25 86.25) (end 165 86.5) (width 0.5) (layer "B.Cu") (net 2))
 (segment (start 152.25 60.25) (end 167 75) (width 0.5) (layer "B.Cu") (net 2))
 (segment (start 167 75) (end 167 84.5) (width 0.5) (layer "B.Cu") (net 2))
 (segment (start 141.5 57) (end 149 57) (width 0.5) (layer "B.Cu") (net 2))
 (segment (start 121.75 58) (end 121.75 61.5) (width 0.5) (layer "B.Cu") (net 2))
 (segment (start 157.5 95.5) (end 147.5 95.5) (width 0.5) (layer "B.Cu") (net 2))
 (segment (start 127.5 53) (end 141.5 53) (width 0.5) (layer "B.Cu") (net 2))
 (segment (start 120 81) (end 120 81.5) (width 0.5) (layer "B.Cu") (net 2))
 (segment (start 167 84.5) (end 165.25 86.25) (width 0.5) (layer "B.Cu") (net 2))
 (segment (start 165 86.5) (end 165 92.5) (width 0.5) (layer "B.Cu") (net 2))
 (segment (start 126.5 53) (end 127.5 53) (width 0.5) (layer "B.Cu") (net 2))
 (segment (start 112.5 73.75) (end 112.5 73.5) (width 0.5) (layer "B.Cu") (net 2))
 (segment (start 112.5 73.5) (end 120 81) (width 0.5) (layer "B.Cu") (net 2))
 (segment (start 145 53) (end 152.25 60.25) (width 0.5) (layer "B.Cu") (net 2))
 (segment (start 124.75 55) (end 124.75 54.75) (width 0.5) (layer "B.Cu") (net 2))
 (segment (start 157.5 95.5) (end 156.25 95.5) (width 0.5) (layer "B.Cu") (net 2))
 (segment (start 121.75 58) (end 124.75 55) (width 0.5) (layer "B.Cu") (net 2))
 (segment (start 165.25 86.25) (end 163 88.5) (width 0.5) (layer "B.Cu") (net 2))
 (segment (start 119.25 61.5) (end 121.75 61.5) (width 0.5) (layer "B.Cu") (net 2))
 (segment (start 127.5 53) (end 129 54.5) (width 0.5) (layer "B.Cu") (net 2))
 (segment (start 124.75 54.75) (end 126.5 53) (width 0.5) (layer "B.Cu") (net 2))
 (segment (start 165 92.5) (end 162 95.5) (width 0.5) (layer "B.Cu") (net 2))
 (segment (start 141.5 57) (end 133.75 64.75) (width 0.5) (layer "B.Cu") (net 2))
 (segment (start 149 57) (end 152.25 60.25) (width 0.5) (layer "B.Cu") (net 2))
 (segment (start 164.5 81.25) (end 152.5 81.25) (width 0.4) (layer "F.Cu") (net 3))
 (segment (start 131.88 82.5) (end 151.25 82.5) (width 0.4) (layer "F.Cu") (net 3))
 (segment (start 151.75 86.5) (end 152.175 86.5) (width 0.2) (layer "F.Cu") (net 3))
 (segment (start 168.5 85.25) (end 164.5 81.25) (width 0.4) (layer "F.Cu") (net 3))
 (segment (start 122.675 85.405) (end 128.975 85.405) (width 0.5) (layer "F.Cu") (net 3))
 (segment (start 154.5 83.5) (end 156 85) (width 0.4) (layer "F.Cu") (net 3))
 (segment (start 128.975 85.405) (end 131.88 82.5) (width 0.4) (layer "F.Cu") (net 3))
 (segment (start 155.25 91.25) (end 157.7 91.25) (width 0.4) (layer "F.Cu") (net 3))
 (segment (start 168.5 94.25) (end 168.5 85.25) (width 0.4) (layer "F.Cu") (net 3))
 (segment (start 165.75 97) (end 168.5 94.25) (width 0.4) (layer "F.Cu") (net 3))
 (segment (start 159 95) (end 159 96) (width 0.4) (layer "F.Cu") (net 3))
 (segment (start 155.1 91.1) (end 155.25 91.25) (width 0.4) (layer "F.Cu") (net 3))
 (segment (start 152.5 81.25) (end 151.25 82.5) (width 0.4) (layer "F.Cu") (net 3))
 (segment (start 155.1 91.1) (end 156.5 92.5) (width 0.4) (layer "F.Cu") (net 3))
 (segment (start 153.225 91.1) (end 155.1 91.1) (width 0.4) (layer "F.Cu") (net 3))
 (segment (start 150.75 85.5) (end 151.75 86.5) (width 0.4) (layer "F.Cu") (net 3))
 (segment (start 159 96) (end 158 97) (width 0.4) (layer "F.Cu") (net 3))
 (segment (start 156 85) (end 157.5 85) (width 0.4) (layer "F.Cu") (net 3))
 (segment (start 152.25 83.5) (end 150.75 85) (width 0.4) (layer "F.Cu") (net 3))
 (segment (start 156.5 92.5) (end 159 95) (width 0.4) (layer "F.Cu") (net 3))
 (segment (start 152.25 83.5) (end 154.5 83.5) (width 0.4) (layer "F.Cu") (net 3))
 (segment (start 158 97) (end 165.75 97) (width 0.4) (layer "F.Cu") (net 3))
 (segment (start 150.75 85) (end 150.75 85.5) (width 0.4) (layer "F.Cu") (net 3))
 (segment (start 151.25 82.5) (end 152.25 83.5) (width 0.4) (layer "F.Cu") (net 3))
 (segment (start 150.75 85.5) (end 149.25 87) (width 0.4) (layer "F.Cu") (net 3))
 (segment (start 142.75 96.25) (end 140.25 96.25) (width 0.4) (layer "F.Cu") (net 12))
 (segment (start 143.5 96.5) (end 143 96.5) (width 0.4) (layer "F.Cu") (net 12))
 (segment (start 143.75 96.75) (end 143.5 96.5) (width 0.4) (layer "F.Cu") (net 12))
 (segment (start 143 96.5) (end 142.75 96.25) (width 0.4) (layer "F.Cu") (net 12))
 (segment (start 145.1 96.75) (end 143.75 96.75) (width 0.4) (layer "F.Cu") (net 12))
 (segment (start 147.5 94.35) (end 145.1 96.75) (width 0.4) (layer "F.Cu") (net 12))
 (segment (start 140.65 93.7) (end 140.25 93.3) (width 0.2) (layer "F.Cu") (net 11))
 (segment (start 142.75 93.7) (end 140.65 93.7) (width 0.4) (layer "F.Cu") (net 11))
 (segment (start 147.5 93.7) (end 142.75 93.7) (width 0.4) (layer "F.Cu") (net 11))
 (segment (start 119.75 88.5) (end 115 83.75) (width 0.4) (layer "F.Cu") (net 4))
 (segment (start 115.5 58) (end 121.25 58) (width 0.4) (layer "F.Cu") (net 4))
 (segment (start 115 58.5) (end 115.5 58) (width 0.4) (layer "F.Cu") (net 4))
 (segment (start 115 81.5) (end 115 58.5) (width 0.4) (layer "F.Cu") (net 4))
 (segment (start 121.25 58) (end 125.25 62) (width 0.4) (layer "F.Cu") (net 4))
 (segment (start 128.34 64.67) (end 128.34 64.07) (width 0.2) (layer "F.Cu") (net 4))
 (segment (start 128.34 64.07) (end 131.41 61) (width 0.4) (layer "F.Cu") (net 4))
 (segment (start 131.41 61) (end 135.5 61) (width 0.4) (layer "F.Cu") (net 4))
 (segment (start 125.3 62.05) (end 125.25 62) (width 0.2) (layer "F.Cu") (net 4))
 (segment (start 135.5 61) (end 141 66.5) (width 0.4) (layer "F.Cu") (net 4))
 (segment (start 141 71.5) (end 135.5 77) (width 0.4) (layer "F.Cu") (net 4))
 (segment (start 135.5 77) (end 119.5 77) (width 0.4) (layer "F.Cu") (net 4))
 (segment (start 122.675 87.705) (end 121.88 88.5) (width 0.4) (layer "F.Cu") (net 4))
 (segment (start 119.5 77) (end 115 81.5) (width 0.4) (layer "F.Cu") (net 4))
 (segment (start 125.3 64.67) (end 125.3 62.05) (width 0.4) (layer "F.Cu") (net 4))
 (segment (start 121.88 88.5) (end 119.75 88.5) (width 0.4) (layer "F.Cu") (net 4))
 (segment (start 141 66.5) (end 141 71.5) (width 0.4) (layer "F.Cu") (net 4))
 (segment (start 115 83.75) (end 115 81.5) (width 0.4) (layer "F.Cu") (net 4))
 (segment (start 127.32 64.07) (end 131.815 59.575) (width 0.2) (layer "F.Cu") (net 1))
 (segment (start 127.32 64.67) (end 127.32 64.07) (width 0.2) (layer "F.Cu") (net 1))
 (segment (start 131.815 59.575) (end 132.25 59.575) (width 0.2) (layer "F.Cu") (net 1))
 (segment (start 126.32 64.67) (end 126.32 59.895) (width 0.2) (layer "F.Cu") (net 5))
 (segment (start 126.32 59.895) (end 126 59.575) (width 0.2) (layer "F.Cu") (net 5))
 (segment (start 147.5 89.8) (end 147.5 87.1) (width 0.2) (layer "F.Cu") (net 6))
 (segment (start 147.5 87.1) (end 147.6 87) (width 0.2) (layer "F.Cu") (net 6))
 (segment (start 153.825 89.2) (end 153.825 86.5) (width 0.2) (layer "F.Cu") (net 7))
 (segment (start 153.225 89.8) (end 153.825 89.2) (width 0.2) (layer "F.Cu") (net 7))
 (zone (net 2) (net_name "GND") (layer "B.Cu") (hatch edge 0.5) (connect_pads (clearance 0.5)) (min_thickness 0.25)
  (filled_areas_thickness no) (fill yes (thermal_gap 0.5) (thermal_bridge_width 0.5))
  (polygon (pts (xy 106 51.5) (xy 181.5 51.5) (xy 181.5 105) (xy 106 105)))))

